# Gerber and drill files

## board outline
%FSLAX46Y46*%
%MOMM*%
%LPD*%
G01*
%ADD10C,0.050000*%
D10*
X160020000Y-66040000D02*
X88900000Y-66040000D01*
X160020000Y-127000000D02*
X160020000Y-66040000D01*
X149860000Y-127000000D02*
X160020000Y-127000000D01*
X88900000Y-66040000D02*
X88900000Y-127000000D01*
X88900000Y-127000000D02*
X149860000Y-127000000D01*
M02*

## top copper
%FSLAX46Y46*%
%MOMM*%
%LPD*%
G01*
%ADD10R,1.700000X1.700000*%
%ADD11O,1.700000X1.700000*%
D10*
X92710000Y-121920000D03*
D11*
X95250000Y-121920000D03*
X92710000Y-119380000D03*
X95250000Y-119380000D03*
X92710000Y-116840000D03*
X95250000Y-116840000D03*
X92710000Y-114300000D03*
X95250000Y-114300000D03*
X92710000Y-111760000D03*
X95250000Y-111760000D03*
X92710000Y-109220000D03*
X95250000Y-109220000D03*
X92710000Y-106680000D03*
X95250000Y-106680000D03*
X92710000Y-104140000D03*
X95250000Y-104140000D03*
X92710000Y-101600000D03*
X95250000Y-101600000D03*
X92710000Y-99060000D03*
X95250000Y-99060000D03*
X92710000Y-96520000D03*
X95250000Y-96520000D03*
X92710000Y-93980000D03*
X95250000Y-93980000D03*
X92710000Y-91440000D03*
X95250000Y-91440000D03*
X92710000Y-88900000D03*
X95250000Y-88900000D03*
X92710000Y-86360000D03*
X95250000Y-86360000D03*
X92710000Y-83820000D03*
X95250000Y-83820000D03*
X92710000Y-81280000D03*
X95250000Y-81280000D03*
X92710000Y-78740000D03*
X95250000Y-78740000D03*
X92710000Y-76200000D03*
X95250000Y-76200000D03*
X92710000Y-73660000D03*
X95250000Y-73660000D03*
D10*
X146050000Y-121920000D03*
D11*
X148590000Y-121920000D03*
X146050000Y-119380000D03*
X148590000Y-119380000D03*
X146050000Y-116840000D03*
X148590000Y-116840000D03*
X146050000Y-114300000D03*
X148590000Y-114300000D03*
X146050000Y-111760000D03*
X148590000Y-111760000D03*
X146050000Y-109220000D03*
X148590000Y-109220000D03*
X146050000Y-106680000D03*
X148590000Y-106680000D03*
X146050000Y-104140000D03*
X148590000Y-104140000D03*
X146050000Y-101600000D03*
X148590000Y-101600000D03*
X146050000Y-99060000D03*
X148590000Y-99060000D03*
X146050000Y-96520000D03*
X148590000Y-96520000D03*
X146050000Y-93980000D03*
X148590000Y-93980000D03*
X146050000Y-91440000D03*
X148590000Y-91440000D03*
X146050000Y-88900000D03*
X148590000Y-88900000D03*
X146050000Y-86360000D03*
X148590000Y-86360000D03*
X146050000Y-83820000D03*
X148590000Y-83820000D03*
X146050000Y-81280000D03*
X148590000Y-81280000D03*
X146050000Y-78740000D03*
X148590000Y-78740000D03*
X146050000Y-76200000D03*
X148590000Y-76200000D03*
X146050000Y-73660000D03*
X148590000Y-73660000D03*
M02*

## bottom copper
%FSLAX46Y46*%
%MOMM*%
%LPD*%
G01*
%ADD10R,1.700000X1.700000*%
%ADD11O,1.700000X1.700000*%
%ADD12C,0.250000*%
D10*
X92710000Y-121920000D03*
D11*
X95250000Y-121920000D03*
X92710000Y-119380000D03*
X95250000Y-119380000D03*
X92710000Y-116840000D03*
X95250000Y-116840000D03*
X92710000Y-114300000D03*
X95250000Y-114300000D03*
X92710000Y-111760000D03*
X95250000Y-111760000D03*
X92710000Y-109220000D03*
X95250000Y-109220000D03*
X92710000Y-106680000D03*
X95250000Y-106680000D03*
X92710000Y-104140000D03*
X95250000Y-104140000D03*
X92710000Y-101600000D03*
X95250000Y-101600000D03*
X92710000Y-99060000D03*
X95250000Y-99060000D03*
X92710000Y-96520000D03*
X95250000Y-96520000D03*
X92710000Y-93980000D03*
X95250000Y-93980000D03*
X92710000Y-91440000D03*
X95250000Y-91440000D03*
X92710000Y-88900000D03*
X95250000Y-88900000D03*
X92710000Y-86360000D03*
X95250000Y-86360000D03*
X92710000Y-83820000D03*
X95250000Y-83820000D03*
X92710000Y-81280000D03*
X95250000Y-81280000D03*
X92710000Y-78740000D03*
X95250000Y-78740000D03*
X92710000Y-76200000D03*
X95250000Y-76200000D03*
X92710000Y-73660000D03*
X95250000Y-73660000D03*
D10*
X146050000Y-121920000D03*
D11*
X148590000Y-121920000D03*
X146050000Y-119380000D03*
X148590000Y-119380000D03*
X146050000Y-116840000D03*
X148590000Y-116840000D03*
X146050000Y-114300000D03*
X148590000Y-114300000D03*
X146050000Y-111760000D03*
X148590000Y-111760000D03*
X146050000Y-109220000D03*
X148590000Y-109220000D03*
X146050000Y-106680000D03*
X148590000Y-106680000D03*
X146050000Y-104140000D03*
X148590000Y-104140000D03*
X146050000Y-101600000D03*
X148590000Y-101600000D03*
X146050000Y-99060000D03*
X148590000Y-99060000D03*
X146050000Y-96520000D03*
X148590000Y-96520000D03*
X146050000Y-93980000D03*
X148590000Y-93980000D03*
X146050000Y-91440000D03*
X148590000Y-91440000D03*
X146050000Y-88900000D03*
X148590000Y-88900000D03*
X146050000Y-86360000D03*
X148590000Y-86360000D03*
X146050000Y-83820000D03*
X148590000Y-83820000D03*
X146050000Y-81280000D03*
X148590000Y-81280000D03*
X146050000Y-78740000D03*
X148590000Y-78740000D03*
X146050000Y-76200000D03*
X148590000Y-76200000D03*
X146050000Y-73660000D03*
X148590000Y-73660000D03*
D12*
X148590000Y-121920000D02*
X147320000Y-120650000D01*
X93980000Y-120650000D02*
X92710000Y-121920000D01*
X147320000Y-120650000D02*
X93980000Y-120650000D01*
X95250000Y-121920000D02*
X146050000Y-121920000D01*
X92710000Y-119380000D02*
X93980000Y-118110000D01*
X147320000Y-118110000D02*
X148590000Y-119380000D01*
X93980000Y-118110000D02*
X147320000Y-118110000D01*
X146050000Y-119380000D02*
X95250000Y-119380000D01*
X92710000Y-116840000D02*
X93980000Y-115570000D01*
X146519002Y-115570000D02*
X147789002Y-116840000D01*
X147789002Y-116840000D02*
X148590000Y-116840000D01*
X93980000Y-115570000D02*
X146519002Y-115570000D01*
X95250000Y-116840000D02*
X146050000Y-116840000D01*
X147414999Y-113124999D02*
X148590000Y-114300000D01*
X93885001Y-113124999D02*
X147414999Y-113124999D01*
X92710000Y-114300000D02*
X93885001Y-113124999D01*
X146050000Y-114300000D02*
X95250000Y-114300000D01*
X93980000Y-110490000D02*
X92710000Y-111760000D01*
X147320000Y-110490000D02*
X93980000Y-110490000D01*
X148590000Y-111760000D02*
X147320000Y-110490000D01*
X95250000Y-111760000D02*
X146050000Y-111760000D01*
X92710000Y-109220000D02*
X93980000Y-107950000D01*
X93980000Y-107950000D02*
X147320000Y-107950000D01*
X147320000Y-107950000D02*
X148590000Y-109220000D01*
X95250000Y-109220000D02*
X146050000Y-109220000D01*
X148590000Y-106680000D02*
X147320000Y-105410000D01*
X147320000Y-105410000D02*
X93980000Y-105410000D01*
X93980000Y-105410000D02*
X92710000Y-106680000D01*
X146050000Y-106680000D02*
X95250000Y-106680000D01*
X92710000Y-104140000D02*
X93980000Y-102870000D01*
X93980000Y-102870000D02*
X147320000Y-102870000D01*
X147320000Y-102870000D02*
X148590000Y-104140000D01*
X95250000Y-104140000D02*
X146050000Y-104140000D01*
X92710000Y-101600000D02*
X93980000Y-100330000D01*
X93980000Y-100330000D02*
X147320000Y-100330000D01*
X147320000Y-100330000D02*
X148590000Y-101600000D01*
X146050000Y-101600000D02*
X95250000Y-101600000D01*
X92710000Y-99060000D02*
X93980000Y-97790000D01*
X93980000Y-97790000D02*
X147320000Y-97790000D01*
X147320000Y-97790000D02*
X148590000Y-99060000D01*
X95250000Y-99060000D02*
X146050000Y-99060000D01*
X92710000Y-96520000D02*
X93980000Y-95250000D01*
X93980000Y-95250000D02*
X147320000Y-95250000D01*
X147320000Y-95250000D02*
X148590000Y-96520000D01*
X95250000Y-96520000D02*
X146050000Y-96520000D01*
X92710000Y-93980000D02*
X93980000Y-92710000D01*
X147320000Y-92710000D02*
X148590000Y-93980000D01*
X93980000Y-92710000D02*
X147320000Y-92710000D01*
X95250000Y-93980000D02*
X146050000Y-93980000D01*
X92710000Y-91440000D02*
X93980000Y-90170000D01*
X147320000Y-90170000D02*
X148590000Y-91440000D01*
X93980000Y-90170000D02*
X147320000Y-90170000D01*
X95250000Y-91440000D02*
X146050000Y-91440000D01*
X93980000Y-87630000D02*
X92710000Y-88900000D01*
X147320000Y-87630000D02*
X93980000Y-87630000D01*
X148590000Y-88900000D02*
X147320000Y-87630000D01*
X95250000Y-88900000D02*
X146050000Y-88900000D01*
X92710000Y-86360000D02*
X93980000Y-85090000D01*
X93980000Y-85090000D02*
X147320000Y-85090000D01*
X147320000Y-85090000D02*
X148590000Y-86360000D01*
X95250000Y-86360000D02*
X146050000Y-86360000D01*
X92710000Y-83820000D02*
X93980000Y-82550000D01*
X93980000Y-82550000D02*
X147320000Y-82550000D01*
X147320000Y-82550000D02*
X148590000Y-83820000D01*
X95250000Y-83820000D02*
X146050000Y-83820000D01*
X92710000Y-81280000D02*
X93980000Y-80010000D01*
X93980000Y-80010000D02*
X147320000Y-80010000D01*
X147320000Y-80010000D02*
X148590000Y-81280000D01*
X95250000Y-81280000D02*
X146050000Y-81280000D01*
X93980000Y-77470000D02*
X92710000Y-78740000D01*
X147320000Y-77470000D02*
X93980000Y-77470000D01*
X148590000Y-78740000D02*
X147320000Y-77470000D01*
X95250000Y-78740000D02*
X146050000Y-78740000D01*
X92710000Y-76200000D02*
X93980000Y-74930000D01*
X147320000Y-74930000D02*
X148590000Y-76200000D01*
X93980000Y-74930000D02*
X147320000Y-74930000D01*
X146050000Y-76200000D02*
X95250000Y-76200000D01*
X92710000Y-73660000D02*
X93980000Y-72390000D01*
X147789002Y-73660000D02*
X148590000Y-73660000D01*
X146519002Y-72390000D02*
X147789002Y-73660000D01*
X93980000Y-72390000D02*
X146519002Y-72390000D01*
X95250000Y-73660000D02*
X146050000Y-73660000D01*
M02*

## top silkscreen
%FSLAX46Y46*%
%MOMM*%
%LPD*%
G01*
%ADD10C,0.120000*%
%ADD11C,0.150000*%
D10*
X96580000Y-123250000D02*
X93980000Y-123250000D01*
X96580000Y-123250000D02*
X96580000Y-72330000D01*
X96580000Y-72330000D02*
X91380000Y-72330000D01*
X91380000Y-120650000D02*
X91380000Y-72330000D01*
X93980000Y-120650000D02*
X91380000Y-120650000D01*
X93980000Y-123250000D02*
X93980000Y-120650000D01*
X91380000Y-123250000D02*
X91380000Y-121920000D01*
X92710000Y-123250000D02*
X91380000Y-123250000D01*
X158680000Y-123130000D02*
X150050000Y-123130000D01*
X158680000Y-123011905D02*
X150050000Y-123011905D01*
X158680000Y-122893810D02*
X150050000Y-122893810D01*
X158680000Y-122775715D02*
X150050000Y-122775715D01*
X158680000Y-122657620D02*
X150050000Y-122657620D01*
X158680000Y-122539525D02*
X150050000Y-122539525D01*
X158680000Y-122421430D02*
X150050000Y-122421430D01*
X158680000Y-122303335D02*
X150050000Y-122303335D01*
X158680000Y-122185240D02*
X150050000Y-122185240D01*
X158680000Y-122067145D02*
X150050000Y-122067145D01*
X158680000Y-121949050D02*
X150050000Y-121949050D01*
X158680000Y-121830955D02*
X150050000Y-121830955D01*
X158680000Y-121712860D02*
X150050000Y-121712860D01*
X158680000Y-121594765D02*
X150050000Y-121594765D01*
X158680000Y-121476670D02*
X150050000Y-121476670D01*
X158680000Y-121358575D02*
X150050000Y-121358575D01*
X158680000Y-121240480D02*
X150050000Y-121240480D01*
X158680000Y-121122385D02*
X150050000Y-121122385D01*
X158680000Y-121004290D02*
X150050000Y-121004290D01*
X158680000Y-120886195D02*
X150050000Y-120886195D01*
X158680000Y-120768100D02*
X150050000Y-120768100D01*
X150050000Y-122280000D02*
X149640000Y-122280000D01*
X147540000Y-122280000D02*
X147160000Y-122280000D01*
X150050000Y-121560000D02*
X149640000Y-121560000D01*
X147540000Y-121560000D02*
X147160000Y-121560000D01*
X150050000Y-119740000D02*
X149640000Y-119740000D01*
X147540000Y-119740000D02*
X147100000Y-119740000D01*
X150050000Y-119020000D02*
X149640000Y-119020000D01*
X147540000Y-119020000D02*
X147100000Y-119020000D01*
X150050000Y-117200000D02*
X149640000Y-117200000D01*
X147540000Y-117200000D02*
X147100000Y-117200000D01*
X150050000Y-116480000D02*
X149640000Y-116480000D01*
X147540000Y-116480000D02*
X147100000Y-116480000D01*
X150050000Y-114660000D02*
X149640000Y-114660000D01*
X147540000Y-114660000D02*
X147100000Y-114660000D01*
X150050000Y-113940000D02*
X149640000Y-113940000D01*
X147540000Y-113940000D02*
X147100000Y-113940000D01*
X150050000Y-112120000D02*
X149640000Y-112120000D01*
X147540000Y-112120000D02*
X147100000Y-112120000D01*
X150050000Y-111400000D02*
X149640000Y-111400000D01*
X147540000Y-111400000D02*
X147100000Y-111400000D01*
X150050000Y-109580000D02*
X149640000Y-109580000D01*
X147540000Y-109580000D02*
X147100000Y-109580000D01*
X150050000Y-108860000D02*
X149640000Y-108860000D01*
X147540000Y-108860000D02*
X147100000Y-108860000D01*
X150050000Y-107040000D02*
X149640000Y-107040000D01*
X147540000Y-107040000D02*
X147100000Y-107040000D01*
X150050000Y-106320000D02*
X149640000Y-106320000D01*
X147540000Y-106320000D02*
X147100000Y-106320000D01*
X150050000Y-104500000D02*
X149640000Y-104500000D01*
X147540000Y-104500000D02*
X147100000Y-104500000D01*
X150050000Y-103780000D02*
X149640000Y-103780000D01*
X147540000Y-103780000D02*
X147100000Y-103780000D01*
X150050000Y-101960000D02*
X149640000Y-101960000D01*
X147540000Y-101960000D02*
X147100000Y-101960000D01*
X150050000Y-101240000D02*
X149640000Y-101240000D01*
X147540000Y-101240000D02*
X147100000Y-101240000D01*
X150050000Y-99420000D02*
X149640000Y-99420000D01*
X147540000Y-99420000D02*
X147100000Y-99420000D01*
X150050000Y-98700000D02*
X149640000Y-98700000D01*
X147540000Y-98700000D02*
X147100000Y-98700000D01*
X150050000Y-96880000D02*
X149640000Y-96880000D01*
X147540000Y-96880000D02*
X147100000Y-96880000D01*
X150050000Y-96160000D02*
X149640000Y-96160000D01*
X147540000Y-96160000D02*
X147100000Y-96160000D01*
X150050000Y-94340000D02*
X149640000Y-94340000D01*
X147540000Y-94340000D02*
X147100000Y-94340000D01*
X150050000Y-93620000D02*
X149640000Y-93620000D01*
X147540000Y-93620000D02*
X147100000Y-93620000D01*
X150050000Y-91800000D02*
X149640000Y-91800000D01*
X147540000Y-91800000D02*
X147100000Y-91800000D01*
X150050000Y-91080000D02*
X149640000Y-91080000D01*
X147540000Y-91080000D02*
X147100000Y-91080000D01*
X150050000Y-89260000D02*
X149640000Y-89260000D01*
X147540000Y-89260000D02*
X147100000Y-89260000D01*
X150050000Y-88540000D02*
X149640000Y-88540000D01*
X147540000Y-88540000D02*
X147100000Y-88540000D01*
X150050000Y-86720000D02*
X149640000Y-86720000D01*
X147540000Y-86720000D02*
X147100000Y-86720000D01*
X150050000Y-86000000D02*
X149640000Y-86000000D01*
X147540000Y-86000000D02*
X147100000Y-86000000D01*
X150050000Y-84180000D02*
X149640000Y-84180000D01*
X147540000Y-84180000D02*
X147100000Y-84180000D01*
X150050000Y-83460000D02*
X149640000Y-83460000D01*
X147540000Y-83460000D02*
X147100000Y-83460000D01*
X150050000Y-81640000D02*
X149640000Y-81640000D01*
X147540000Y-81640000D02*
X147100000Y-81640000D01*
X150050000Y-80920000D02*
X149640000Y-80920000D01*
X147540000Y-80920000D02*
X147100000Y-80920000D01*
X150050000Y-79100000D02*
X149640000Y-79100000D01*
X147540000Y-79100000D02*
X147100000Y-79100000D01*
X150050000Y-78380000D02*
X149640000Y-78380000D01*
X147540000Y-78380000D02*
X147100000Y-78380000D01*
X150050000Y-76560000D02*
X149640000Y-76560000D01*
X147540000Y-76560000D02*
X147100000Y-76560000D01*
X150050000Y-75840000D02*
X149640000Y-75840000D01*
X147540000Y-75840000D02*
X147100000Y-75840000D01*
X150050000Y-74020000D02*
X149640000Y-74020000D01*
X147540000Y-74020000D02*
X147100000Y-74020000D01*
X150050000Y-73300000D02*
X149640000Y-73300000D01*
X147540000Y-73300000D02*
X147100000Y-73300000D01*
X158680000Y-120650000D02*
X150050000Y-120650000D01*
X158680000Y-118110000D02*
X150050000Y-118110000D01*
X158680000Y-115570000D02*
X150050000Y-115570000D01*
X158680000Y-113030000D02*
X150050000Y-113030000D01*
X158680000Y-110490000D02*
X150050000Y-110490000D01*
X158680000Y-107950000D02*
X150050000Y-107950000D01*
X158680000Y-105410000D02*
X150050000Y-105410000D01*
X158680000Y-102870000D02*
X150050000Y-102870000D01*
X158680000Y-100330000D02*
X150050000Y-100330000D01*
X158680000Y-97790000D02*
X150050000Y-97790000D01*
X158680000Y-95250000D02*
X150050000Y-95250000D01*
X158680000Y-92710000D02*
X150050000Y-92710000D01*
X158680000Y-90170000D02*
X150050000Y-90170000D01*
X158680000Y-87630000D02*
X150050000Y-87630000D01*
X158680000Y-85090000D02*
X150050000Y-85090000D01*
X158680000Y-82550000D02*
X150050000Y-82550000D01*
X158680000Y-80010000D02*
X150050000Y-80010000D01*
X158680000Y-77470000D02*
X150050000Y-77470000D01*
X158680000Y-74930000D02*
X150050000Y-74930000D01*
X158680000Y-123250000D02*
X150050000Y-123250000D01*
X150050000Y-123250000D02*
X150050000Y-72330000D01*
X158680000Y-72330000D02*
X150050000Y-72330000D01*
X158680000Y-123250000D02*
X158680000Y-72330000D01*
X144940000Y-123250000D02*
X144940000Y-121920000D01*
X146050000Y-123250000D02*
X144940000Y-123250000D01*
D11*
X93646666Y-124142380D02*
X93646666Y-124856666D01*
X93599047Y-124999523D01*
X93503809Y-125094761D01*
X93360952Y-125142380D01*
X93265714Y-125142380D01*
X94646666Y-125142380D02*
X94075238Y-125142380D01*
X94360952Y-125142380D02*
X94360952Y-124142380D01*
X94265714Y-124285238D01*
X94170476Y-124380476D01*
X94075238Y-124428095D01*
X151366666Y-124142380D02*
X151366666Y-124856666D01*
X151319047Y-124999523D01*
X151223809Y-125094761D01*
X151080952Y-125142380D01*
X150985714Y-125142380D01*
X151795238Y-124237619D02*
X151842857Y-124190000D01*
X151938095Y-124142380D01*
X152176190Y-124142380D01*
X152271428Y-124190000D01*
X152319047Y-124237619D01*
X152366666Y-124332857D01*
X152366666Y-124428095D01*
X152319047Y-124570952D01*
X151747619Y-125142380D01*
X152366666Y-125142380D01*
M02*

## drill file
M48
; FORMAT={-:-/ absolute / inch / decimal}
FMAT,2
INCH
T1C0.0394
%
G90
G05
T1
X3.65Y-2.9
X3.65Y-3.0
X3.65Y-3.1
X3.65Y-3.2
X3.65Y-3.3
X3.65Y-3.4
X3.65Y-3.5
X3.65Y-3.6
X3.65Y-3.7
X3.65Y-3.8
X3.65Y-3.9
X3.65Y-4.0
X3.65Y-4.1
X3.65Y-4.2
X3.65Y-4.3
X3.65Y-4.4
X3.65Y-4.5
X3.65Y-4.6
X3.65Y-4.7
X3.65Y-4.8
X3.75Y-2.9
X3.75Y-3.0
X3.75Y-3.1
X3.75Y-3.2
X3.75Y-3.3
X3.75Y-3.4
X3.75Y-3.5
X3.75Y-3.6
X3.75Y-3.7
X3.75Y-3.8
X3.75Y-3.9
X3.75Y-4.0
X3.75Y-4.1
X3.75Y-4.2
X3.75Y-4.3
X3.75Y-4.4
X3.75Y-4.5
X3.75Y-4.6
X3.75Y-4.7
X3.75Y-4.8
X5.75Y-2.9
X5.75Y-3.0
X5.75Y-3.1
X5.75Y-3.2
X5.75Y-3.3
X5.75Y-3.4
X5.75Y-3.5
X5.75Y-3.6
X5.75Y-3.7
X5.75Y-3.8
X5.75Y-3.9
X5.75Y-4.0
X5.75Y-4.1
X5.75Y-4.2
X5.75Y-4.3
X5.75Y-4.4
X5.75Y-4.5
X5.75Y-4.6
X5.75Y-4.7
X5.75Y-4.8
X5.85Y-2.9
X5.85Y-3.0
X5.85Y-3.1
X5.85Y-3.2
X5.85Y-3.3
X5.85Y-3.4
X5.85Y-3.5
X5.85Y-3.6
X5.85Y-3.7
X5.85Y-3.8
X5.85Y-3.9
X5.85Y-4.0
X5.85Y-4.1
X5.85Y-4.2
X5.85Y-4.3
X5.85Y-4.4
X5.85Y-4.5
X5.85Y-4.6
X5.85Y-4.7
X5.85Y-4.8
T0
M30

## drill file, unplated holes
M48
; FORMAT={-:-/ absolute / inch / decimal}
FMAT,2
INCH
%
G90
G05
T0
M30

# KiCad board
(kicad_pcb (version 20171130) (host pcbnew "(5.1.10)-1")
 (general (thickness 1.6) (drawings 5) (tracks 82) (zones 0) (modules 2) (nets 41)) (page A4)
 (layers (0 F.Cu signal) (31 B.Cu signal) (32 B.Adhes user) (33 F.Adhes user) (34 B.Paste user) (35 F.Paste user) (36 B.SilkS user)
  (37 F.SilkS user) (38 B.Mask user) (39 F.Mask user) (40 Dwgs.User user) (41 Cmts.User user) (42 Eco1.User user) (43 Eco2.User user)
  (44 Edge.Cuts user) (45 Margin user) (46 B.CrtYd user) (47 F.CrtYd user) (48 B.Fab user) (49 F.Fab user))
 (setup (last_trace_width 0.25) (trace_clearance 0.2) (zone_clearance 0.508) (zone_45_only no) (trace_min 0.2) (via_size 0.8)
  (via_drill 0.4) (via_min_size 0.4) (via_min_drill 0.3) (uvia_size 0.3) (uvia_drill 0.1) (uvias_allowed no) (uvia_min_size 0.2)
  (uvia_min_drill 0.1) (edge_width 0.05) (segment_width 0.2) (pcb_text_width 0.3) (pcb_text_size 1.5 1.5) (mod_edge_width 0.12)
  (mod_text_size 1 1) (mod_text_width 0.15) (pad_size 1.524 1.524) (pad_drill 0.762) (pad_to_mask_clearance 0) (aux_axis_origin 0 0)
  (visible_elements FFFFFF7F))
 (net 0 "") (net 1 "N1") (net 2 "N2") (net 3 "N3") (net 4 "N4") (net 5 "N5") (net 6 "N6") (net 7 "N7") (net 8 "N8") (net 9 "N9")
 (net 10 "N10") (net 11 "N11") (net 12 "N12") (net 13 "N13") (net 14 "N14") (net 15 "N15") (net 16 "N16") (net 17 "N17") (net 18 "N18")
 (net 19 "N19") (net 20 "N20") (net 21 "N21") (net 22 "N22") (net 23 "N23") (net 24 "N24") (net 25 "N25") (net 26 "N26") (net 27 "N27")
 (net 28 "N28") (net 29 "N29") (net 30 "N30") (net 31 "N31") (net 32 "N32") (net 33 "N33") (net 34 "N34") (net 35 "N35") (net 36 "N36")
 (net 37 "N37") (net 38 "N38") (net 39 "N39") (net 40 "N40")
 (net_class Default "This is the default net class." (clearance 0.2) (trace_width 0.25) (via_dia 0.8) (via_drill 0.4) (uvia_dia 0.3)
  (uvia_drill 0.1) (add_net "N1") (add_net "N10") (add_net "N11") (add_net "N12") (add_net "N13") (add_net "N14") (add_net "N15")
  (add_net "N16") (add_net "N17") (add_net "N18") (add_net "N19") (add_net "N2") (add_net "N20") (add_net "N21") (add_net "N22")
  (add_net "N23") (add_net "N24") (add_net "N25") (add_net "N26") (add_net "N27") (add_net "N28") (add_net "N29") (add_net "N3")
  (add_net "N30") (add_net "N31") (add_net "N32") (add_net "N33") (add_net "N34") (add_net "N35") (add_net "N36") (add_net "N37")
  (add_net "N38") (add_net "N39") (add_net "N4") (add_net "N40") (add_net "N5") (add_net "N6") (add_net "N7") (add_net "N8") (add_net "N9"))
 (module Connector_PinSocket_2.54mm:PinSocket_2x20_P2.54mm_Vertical (layer F.Cu) (at 92.71 121.92 180)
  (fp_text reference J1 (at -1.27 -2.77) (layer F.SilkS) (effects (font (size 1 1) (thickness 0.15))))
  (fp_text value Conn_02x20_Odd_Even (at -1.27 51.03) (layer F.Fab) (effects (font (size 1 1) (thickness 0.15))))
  (fp_line (start 0 -1.33) (end 1.33 -1.33) (layer F.SilkS) (width 0.12))
  (fp_line (start 1.33 -1.33) (end 1.33 0) (layer F.SilkS) (width 0.12))
  (fp_line (start -1.27 -1.33) (end -1.27 1.27) (layer F.SilkS) (width 0.12))
  (fp_line (start -1.27 1.27) (end 1.33 1.27) (layer F.SilkS) (width 0.12))
  (fp_line (start 1.33 1.27) (end 1.33 49.59) (layer F.SilkS) (width 0.12))
  (fp_line (start -3.87 49.59) (end 1.33 49.59) (layer F.SilkS) (width 0.12))
  (fp_line (start -3.87 -1.33) (end -3.87 49.59) (layer F.SilkS) (width 0.12))
  (fp_line (start -3.87 -1.33) (end -1.27 -1.33) (layer F.SilkS) (width 0.12))
  (pad 1 thru_hole rect (at 0 0 180) (size 1.7 1.7) (drill 1) (layers *.Cu *.Mask) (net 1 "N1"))
  (pad 2 thru_hole oval (at -2.54 0 180) (size 1.7 1.7) (drill 1) (layers *.Cu *.Mask) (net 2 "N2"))
  (pad 3 thru_hole oval (at 0 2.54 180) (size 1.7 1.7) (drill 1) (layers *.Cu *.Mask) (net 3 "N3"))
  (pad 4 thru_hole oval (at -2.54 2.54 180) (size 1.7 1.7) (drill 1) (layers *.Cu *.Mask) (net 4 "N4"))
  (pad 5 thru_hole oval (at 0 5.08 180) (size 1.7 1.7) (drill 1) (layers *.Cu *.Mask) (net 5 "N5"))
  (pad 6 thru_hole oval (at -2.54 5.08 180) (size 1.7 1.7) (drill 1) (layers *.Cu *.Mask) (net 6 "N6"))
  (pad 7 thru_hole oval (at 0 7.62 180) (size 1.7 1.7) (drill 1) (layers *.Cu *.Mask) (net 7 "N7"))
  (pad 8 thru_hole oval (at -2.54 7.62 180) (size 1.7 1.7) (drill 1) (layers *.Cu *.Mask) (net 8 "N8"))
  (pad 9 thru_hole oval (at 0 10.16 180) (size 1.7 1.7) (drill 1) (layers *.Cu *.Mask) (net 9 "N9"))
  (pad 10 thru_hole oval (at -2.54 10.16 180) (size 1.7 1.7) (drill 1) (layers *.Cu *.Mask) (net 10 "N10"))
  (pad 11 thru_hole oval (at 0 12.7 180) (size 1.7 1.7) (drill 1) (layers *.Cu *.Mask) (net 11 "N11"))
  (pad 12 thru_hole oval (at -2.54 12.7 180) (size 1.7 1.7) (drill 1) (layers *.Cu *.Mask) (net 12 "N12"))
  (pad 13 thru_hole oval (at 0 15.24 180) (size 1.7 1.7) (drill 1) (layers *.Cu *.Mask) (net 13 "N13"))
  (pad 14 thru_hole oval (at -2.54 15.24 180) (size 1.7 1.7) (drill 1) (layers *.Cu *.Mask) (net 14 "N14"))
  (pad 15 thru_hole oval (at 0 17.78 180) (size 1.7 1.7) (drill 1) (layers *.Cu *.Mask) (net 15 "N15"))
  (pad 16 thru_hole oval (at -2.54 17.78 180) (size 1.7 1.7) (drill 1) (layers *.Cu *.Mask) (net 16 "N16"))
  (pad 17 thru_hole oval (at 0 20.32 180) (size 1.7 1.7) (drill 1) (layers *.Cu *.Mask) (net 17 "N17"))
  (pad 18 thru_hole oval (at -2.54 20.32 180) (size 1.7 1.7) (drill 1) (layers *.Cu *.Mask) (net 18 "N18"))
  (pad 19 thru_hole oval (at 0 22.86 180) (size 1.7 1.7) (drill 1) (layers *.Cu *.Mask) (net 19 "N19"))
  (pad 20 thru_hole oval (at -2.54 22.86 180) (size 1.7 1.7) (drill 1) (layers *.Cu *.Mask) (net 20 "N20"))
  (pad 21 thru_hole oval (at 0 25.4 180) (size 1.7 1.7) (drill 1) (layers *.Cu *.Mask) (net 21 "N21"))
  (pad 22 thru_hole oval (at -2.54 25.4 180) (size 1.7 1.7) (drill 1) (layers *.Cu *.Mask) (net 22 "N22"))
  (pad 23 thru_hole oval (at 0 27.94 180) (size 1.7 1.7) (drill 1) (layers *.Cu *.Mask) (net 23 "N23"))
  (pad 24 thru_hole oval (at -2.54 27.94 180) (size 1.7 1.7) (drill 1) (layers *.Cu *.Mask) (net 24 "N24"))
  (pad 25 thru_hole oval (at 0 30.48 180) (size 1.7 1.7) (drill 1) (layers *.Cu *.Mask) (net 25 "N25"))
  (pad 26 thru_hole oval (at -2.54 30.48 180) (size 1.7 1.7) (drill 1) (layers *.Cu *.Mask) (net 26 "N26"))
  (pad 27 thru_hole oval (at 0 33.02 180) (size 1.7 1.7) (drill 1) (layers *.Cu *.Mask) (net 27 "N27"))
  (pad 28 thru_hole oval (at -2.54 33.02 180) (size 1.7 1.7) (drill 1) (layers *.Cu *.Mask) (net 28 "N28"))
  (pad 29 thru_hole oval (at 0 35.56 180) (size 1.7 1.7) (drill 1) (layers *.Cu *.Mask) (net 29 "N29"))
  (pad 30 thru_hole oval (at -2.54 35.56 180) (size 1.7 1.7) (drill 1) (layers *.Cu *.Mask) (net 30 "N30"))
  (pad 31 thru_hole oval (at 0 38.1 180) (size 1.7 1.7) (drill 1) (layers *.Cu *.Mask) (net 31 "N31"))
  (pad 32 thru_hole oval (at -2.54 38.1 180) (size 1.7 1.7) (drill 1) (layers *.Cu *.Mask) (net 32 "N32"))
  (pad 33 thru_hole oval (at 0 40.64 180) (size 1.7 1.7) (drill 1) (layers *.Cu *.Mask) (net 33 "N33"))
  (pad 34 thru_hole oval (at -2.54 40.64 180) (size 1.7 1.7) (drill 1) (layers *.Cu *.Mask) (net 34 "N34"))
  (pad 35 thru_hole oval (at 0 43.18 180) (size 1.7 1.7) (drill 1) (layers *.Cu *.Mask) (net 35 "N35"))
  (pad 36 thru_hole oval (at -2.54 43.18 180) (size 1.7 1.7) (drill 1) (layers *.Cu *.Mask) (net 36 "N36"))
  (pad 37 thru_hole oval (at 0 45.72 180) (size 1.7 1.7) (drill 1) (layers *.Cu *.Mask) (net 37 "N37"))
  (pad 38 thru_hole oval (at -2.54 45.72 180) (size 1.7 1.7) (drill 1) (layers *.Cu *.Mask) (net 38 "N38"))
  (pad 39 thru_hole oval (at 0 48.26 180) (size 1.7 1.7) (drill 1) (layers *.Cu *.Mask) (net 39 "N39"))
  (pad 40 thru_hole oval (at -2.54 48.26 180) (size 1.7 1.7) (drill 1) (layers *.Cu *.Mask) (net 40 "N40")))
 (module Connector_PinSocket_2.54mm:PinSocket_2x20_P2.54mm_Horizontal (layer F.Cu) (at 146.05 121.92 180)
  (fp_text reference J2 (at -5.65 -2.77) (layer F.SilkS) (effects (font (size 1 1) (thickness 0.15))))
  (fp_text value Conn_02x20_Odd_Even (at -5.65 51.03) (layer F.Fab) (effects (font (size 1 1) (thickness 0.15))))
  (fp_line (start 0 -1.33) (end 1.11 -1.33) (layer F.SilkS) (width 0.12))
  (fp_line (start 1.11 -1.33) (end 1.11 0) (layer F.SilkS) (width 0.12))
  (fp_line (start -12.63 -1.33) (end -12.63 49.59) (layer F.SilkS) (width 0.12))
  (fp_line (start -12.63 49.59) (end -4 49.59) (layer F.SilkS) (width 0.12))
  (fp_line (start -4 -1.33) (end -4 49.59) (layer F.SilkS) (width 0.12))
  (fp_line (start -12.63 -1.33) (end -4 -1.33) (layer F.SilkS) (width 0.12))
  (fp_line (start -12.63 46.99) (end -4 46.99) (layer F.SilkS) (width 0.12))
  (fp_line (start -12.63 44.45) (end -4 44.45) (layer F.SilkS) (width 0.12))
  (fp_line (start -12.63 41.91) (end -4 41.91) (layer F.SilkS) (width 0.12))
  (fp_line (start -12.63 39.37) (end -4 39.37) (layer F.SilkS) (width 0.12))
  (fp_line (start -12.63 36.83) (end -4 36.83) (layer F.SilkS) (width 0.12))
  (fp_line (start -12.63 34.29) (end -4 34.29) (layer F.SilkS) (width 0.12))
  (fp_line (start -12.63 31.75) (end -4 31.75) (layer F.SilkS) (width 0.12))
  (fp_line (start -12.63 29.21) (end -4 29.21) (layer F.SilkS) (width 0.12))
  (fp_line (start -12.63 26.67) (end -4 26.67) (layer F.SilkS) (width 0.12))
  (fp_line (start -12.63 24.13) (end -4 24.13) (layer F.SilkS) (width 0.12))
  (fp_line (start -12.63 21.59) (end -4 21.59) (layer F.SilkS) (width 0.12))
  (fp_line (start -12.63 19.05) (end -4 19.05) (layer F.SilkS) (width 0.12))
  (fp_line (start -12.63 16.51) (end -4 16.51) (layer F.SilkS) (width 0.12))
  (fp_line (start -12.63 13.97) (end -4 13.97) (layer F.SilkS) (width 0.12))
  (fp_line (start -12.63 11.43) (end -4 11.43) (layer F.SilkS) (width 0.12))
  (fp_line (start -12.63 8.89) (end -4 8.89) (layer F.SilkS) (width 0.12))
  (fp_line (start -12.63 6.35) (end -4 6.35) (layer F.SilkS) (width 0.12))
  (fp_line (start -12.63 3.81) (end -4 3.81) (layer F.SilkS) (width 0.12))
  (fp_line (start -12.63 1.27) (end -4 1.27) (layer F.SilkS) (width 0.12))
  (fp_line (start -1.49 48.62) (end -1.05 48.62) (layer F.SilkS) (width 0.12))
  (fp_line (start -4 48.62) (end -3.59 48.62) (layer F.SilkS) (width 0.12))
  (fp_line (start -1.49 47.9) (end -1.05 47.9) (layer F.SilkS) (width 0.12))
  (fp_line (start -4 47.9) (end -3.59 47.9) (layer F.SilkS) (width 0.12))
  (fp_line (start -1.49 46.08) (end -1.05 46.08) (layer F.SilkS) (width 0.12))
  (fp_line (start -4 46.08) (end -3.59 46.08) (layer F.SilkS) (width 0.12))
  (fp_line (start -1.49 45.36) (end -1.05 45.36) (layer F.SilkS) (width 0.12))
  (fp_line (start -4 45.36) (end -3.59 45.36) (layer F.SilkS) (width 0.12))
  (fp_line (start -1.49 43.54) (end -1.05 43.54) (layer F.SilkS) (width 0.12))
  (fp_line (start -4 43.54) (end -3.59 43.54) (layer F.SilkS) (width 0.12))
  (fp_line (start -1.49 42.82) (end -1.05 42.82) (layer F.SilkS) (width 0.12))
  (fp_line (start -4 42.82) (end -3.59 42.82) (layer F.SilkS) (width 0.12))
  (fp_line (start -1.49 41) (end -1.05 41) (layer F.SilkS) (width 0.12))
  (fp_line (start -4 41) (end -3.59 41) (layer F.SilkS) (width 0.12))
  (fp_line (start -1.49 40.28) (end -1.05 40.28) (layer F.SilkS) (width 0.12))
  (fp_line (start -4 40.28) (end -3.59 40.28) (layer F.SilkS) (width 0.12))
  (fp_line (start -1.49 38.46) (end -1.05 38.46) (layer F.SilkS) (width 0.12))
  (fp_line (start -4 38.46) (end -3.59 38.46) (layer F.SilkS) (width 0.12))
  (fp_line (start -1.49 37.74) (end -1.05 37.74) (layer F.SilkS) (width 0.12))
  (fp_line (start -4 37.74) (end -3.59 37.74) (layer F.SilkS) (width 0.12))
  (fp_line (start -1.49 35.92) (end -1.05 35.92) (layer F.SilkS) (width 0.12))
  (fp_line (start -4 35.92) (end -3.59 35.92) (layer F.SilkS) (width 0.12))
  (fp_line (start -1.49 35.2) (end -1.05 35.2) (layer F.SilkS) (width 0.12))
  (fp_line (start -4 35.2) (end -3.59 35.2) (layer F.SilkS) (width 0.12))
  (fp_line (start -1.49 33.38) (end -1.05 33.38) (layer F.SilkS) (width 0.12))
  (fp_line (start -4 33.38) (end -3.59 33.38) (layer F.SilkS) (width 0.12))
  (fp_line (start -1.49 32.66) (end -1.05 32.66) (layer F.SilkS) (width 0.12))
  (fp_line (start -4 32.66) (end -3.59 32.66) (layer F.SilkS) (width 0.12))
  (fp_line (start -1.49 30.84) (end -1.05 30.84) (layer F.SilkS) (width 0.12))
  (fp_line (start -4 30.84) (end -3.59 30.84) (layer F.SilkS) (width 0.12))
  (fp_line (start -1.49 30.12) (end -1.05 30.12) (layer F.SilkS) (width 0.12))
  (fp_line (start -4 30.12) (end -3.59 30.12) (layer F.SilkS) (width 0.12))
  (fp_line (start -1.49 28.3) (end -1.05 28.3) (layer F.SilkS) (width 0.12))
  (fp_line (start -4 28.3) (end -3.59 28.3) (layer F.SilkS) (width 0.12))
  (fp_line (start -1.49 27.58) (end -1.05 27.58) (layer F.SilkS) (width 0.12))
  (fp_line (start -4 27.58) (end -3.59 27.58) (layer F.SilkS) (width 0.12))
  (fp_line (start -1.49 25.76) (end -1.05 25.76) (layer F.SilkS) (width 0.12))
  (fp_line (start -4 25.76) (end -3.59 25.76) (layer F.SilkS) (width 0.12))
  (fp_line (start -1.49 25.04) (end -1.05 25.04) (layer F.SilkS) (width 0.12))
  (fp_line (start -4 25.04) (end -3.59 25.04) (layer F.SilkS) (width 0.12))
  (fp_line (start -1.49 23.22) (end -1.05 23.22) (layer F.SilkS) (width 0.12))
  (fp_line (start -4 23.22) (end -3.59 23.22) (layer F.SilkS) (width 0.12))
  (fp_line (start -1.49 22.5) (end -1.05 22.5) (layer F.SilkS) (width 0.12))
  (fp_line (start -4 22.5) (end -3.59 22.5) (layer F.SilkS) (width 0.12))
  (fp_line (start -1.49 20.68) (end -1.05 20.68) (layer F.SilkS) (width 0.12))
  (fp_line (start -4 20.68) (end -3.59 20.68) (layer F.SilkS) (width 0.12))
  (fp_line (start -1.49 19.96) (end -1.05 19.96) (layer F.SilkS) (width 0.12))
  (fp_line (start -4 19.96) (end -3.59 19.96) (layer F.SilkS) (width 0.12))
  (fp_line (start -1.49 18.14) (end -1.05 18.14) (layer F.SilkS) (width 0.12))
  (fp_line (start -4 18.14) (end -3.59 18.14) (layer F.SilkS) (width 0.12))
  (fp_line (start -1.49 17.42) (end -1.05 17.42) (layer F.SilkS) (width 0.12))
  (fp_line (start -4 17.42) (end -3.59 17.42) (layer F.SilkS) (width 0.12))
  (fp_line (start -1.49 15.6) (end -1.05 15.6) (layer F.SilkS) (width 0.12))
  (fp_line (start -4 15.6) (end -3.59 15.6) (layer F.SilkS) (width 0.12))
  (fp_line (start -1.49 14.88) (end -1.05 14.88) (layer F.SilkS) (width 0.12))
  (fp_line (start -4 14.88) (end -3.59 14.88) (layer F.SilkS) (width 0.12))
  (fp_line (start -1.49 13.06) (end -1.05 13.06) (layer F.SilkS) (width 0.12))
  (fp_line (start -4 13.06) (end -3.59 13.06) (layer F.SilkS) (width 0.12))
  (fp_line (start -1.49 12.34) (end -1.05 12.34) (layer F.SilkS) (width 0.12))
  (fp_line (start -4 12.34) (end -3.59 12.34) (layer F.SilkS) (width 0.12))
  (fp_line (start -1.49 10.52) (end -1.05 10.52) (layer F.SilkS) (width 0.12))
  (fp_line (start -4 10.52) (end -3.59 10.52) (layer F.SilkS) (width 0.12))
  (fp_line (start -1.49 9.8) (end -1.05 9.8) (layer F.SilkS) (width 0.12))
  (fp_line (start -4 9.8) (end -3.59 9.8) (layer F.SilkS) (width 0.12))
  (fp_line (start -1.49 7.98) (end -1.05 7.98) (layer F.SilkS) (width 0.12))
  (fp_line (start -4 7.98) (end -3.59 7.98) (layer F.SilkS) (width 0.12))
  (fp_line (start -1.49 7.26) (end -1.05 7.26) (layer F.SilkS) (width 0.12))
  (fp_line (start -4 7.26) (end -3.59 7.26) (layer F.SilkS) (width 0.12))
  (fp_line (start -1.49 5.44) (end -1.05 5.44) (layer F.SilkS) (width 0.12))
  (fp_line (start -4 5.44) (end -3.59 5.44) (layer F.SilkS) (width 0.12))
  (fp_line (start -1.49 4.72) (end -1.05 4.72) (layer F.SilkS) (width 0.12))
  (fp_line (start -4 4.72) (end -3.59 4.72) (layer F.SilkS) (width 0.12))
  (fp_line (start -1.49 2.9) (end -1.05 2.9) (layer F.SilkS) (width 0.12))
  (fp_line (start -4 2.9) (end -3.59 2.9) (layer F.SilkS) (width 0.12))
  (fp_line (start -1.49 2.18) (end -1.05 2.18) (layer F.SilkS) (width 0.12))
  (fp_line (start -4 2.18) (end -3.59 2.18) (layer F.SilkS) (width 0.12))
  (fp_line (start -1.49 0.36) (end -1.11 0.36) (layer F.SilkS) (width 0.12))
  (fp_line (start -4 0.36) (end -3.59 0.36) (layer F.SilkS) (width 0.12))
  (fp_line (start -1.49 -0.36) (end -1.11 -0.36) (layer F.SilkS) (width 0.12))
  (fp_line (start -4 -0.36) (end -3.59 -0.36) (layer F.SilkS) (width 0.12))
  (fp_line (start -12.63 1.1519) (end -4 1.1519) (layer F.SilkS) (width 0.12))
  (fp_line (start -12.63 1.033805) (end -4 1.033805) (layer F.SilkS) (width 0.12))
  (fp_line (start -12.63 0.91571) (end -4 0.91571) (layer F.SilkS) (width 0.12))
  (fp_line (start -12.63 0.797615) (end -4 0.797615) (layer F.SilkS) (width 0.12))
  (fp_line (start -12.63 0.67952) (end -4 0.67952) (layer F.SilkS) (width 0.12))
  (fp_line (start -12.63 0.561425) (end -4 0.561425) (layer F.SilkS) (width 0.12))
  (fp_line (start -12.63 0.44333) (end -4 0.44333) (layer F.SilkS) (width 0.12))
  (fp_line (start -12.63 0.325235) (end -4 0.325235) (layer F.SilkS) (width 0.12))
  (fp_line (start -12.63 0.20714) (end -4 0.20714) (layer F.SilkS) (width 0.12))
  (fp_line (start -12.63 0.089045) (end -4 0.089045) (layer F.SilkS) (width 0.12))
  (fp_line (start -12.63 -0.02905) (end -4 -0.02905) (layer F.SilkS) (width 0.12))
  (fp_line (start -12.63 -0.147145) (end -4 -0.147145) (layer F.SilkS) (width 0.12))
  (fp_line (start -12.63 -0.26524) (end -4 -0.26524) (layer F.SilkS) (width 0.12))
  (fp_line (start -12.63 -0.383335) (end -4 -0.383335) (layer F.SilkS) (width 0.12))
  (fp_line (start -12.63 -0.50143) (end -4 -0.50143) (layer F.SilkS) (width 0.12))
  (fp_line (start -12.63 -0.619525) (end -4 -0.619525) (layer F.SilkS) (width 0.12))
  (fp_line (start -12.63 -0.73762) (end -4 -0.73762) (layer F.SilkS) (width 0.12))
  (fp_line (start -12.63 -0.855715) (end -4 -0.855715) (layer F.SilkS) (width 0.12))
  (fp_line (start -12.63 -0.97381) (end -4 -0.97381) (layer F.SilkS) (width 0.12))
  (fp_line (start -12.63 -1.091905) (end -4 -1.091905) (layer F.SilkS) (width 0.12))
  (fp_line (start -12.63 -1.21) (end -4 -1.21) (layer F.SilkS) (width 0.12))
  (pad 1 thru_hole rect (at 0 0 180) (size 1.7 1.7) (drill 1) (layers *.Cu *.Mask) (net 2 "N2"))
  (pad 2 thru_hole oval (at -2.54 0 180) (size 1.7 1.7) (drill 1) (layers *.Cu *.Mask) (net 1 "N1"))
  (pad 3 thru_hole oval (at 0 2.54 180) (size 1.7 1.7) (drill 1) (layers *.Cu *.Mask) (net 4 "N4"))
  (pad 4 thru_hole oval (at -2.54 2.54 180) (size 1.7 1.7) (drill 1) (layers *.Cu *.Mask) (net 3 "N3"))
  (pad 5 thru_hole oval (at 0 5.08 180) (size 1.7 1.7) (drill 1) (layers *.Cu *.Mask) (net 6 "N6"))
  (pad 6 thru_hole oval (at -2.54 5.08 180) (size 1.7 1.7) (drill 1) (layers *.Cu *.Mask) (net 5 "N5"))
  (pad 7 thru_hole oval (at 0 7.62 180) (size 1.7 1.7) (drill 1) (layers *.Cu *.Mask) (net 8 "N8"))
  (pad 8 thru_hole oval (at -2.54 7.62 180) (size 1.7 1.7) (drill 1) (layers *.Cu *.Mask) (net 7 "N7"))
  (pad 9 thru_hole oval (at 0 10.16 180) (size 1.7 1.7) (drill 1) (layers *.Cu *.Mask) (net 10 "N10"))
  (pad 10 thru_hole oval (at -2.54 10.16 180) (size 1.7 1.7) (drill 1) (layers *.Cu *.Mask) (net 9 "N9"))
  (pad 11 thru_hole oval (at 0 12.7 180) (size 1.7 1.7) (drill 1) (layers *.Cu *.Mask) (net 12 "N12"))
  (pad 12 thru_hole oval (at -2.54 12.7 180) (size 1.7 1.7) (drill 1) (layers *.Cu *.Mask) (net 11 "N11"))
  (pad 13 thru_hole oval (at 0 15.24 180) (size 1.7 1.7) (drill 1) (layers *.Cu *.Mask) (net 14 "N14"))
  (pad 14 thru_hole oval (at -2.54 15.24 180) (size 1.7 1.7) (drill 1) (layers *.Cu *.Mask) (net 13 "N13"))
  (pad 15 thru_hole oval (at 0 17.78 180) (size 1.7 1.7) (drill 1) (layers *.Cu *.Mask) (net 16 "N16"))
  (pad 16 thru_hole oval (at -2.54 17.78 180) (size 1.7 1.7) (drill 1) (layers *.Cu *.Mask) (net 15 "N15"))
  (pad 17 thru_hole oval (at 0 20.32 180) (size 1.7 1.7) (drill 1) (layers *.Cu *.Mask) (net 18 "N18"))
  (pad 18 thru_hole oval (at -2.54 20.32 180) (size 1.7 1.7) (drill 1) (layers *.Cu *.Mask) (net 17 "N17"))
  (pad 19 thru_hole oval (at 0 22.86 180) (size 1.7 1.7) (drill 1) (layers *.Cu *.Mask) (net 20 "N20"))
  (pad 20 thru_hole oval (at -2.54 22.86 180) (size 1.7 1.7) (drill 1) (layers *.Cu *.Mask) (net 19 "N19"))
  (pad 21 thru_hole oval (at 0 25.4 180) (size 1.7 1.7) (drill 1) (layers *.Cu *.Mask) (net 22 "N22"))
  (pad 22 thru_hole oval (at -2.54 25.4 180) (size 1.7 1.7) (drill 1) (layers *.Cu *.Mask) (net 21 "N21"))
  (pad 23 thru_hole oval (at 0 27.94 180) (size 1.7 1.7) (drill 1) (layers *.Cu *.Mask) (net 24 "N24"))
  (pad 24 thru_hole oval (at -2.54 27.94 180) (size 1.7 1.7) (drill 1) (layers *.Cu *.Mask) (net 23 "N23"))
  (pad 25 thru_hole oval (at 0 30.48 180) (size 1.7 1.7) (drill 1) (layers *.Cu *.Mask) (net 26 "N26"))
  (pad 26 thru_hole oval (at -2.54 30.48 180) (size 1.7 1.7) (drill 1) (layers *.Cu *.Mask) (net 25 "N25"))
  (pad 27 thru_hole oval (at 0 33.02 180) (size 1.7 1.7) (drill 1) (layers *.Cu *.Mask) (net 28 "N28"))
  (pad 28 thru_hole oval (at -2.54 33.02 180) (size 1.7 1.7) (drill 1) (layers *.Cu *.Mask) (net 27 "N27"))
  (pad 29 thru_hole oval (at 0 35.56 180) (size 1.7 1.7) (drill 1) (layers *.Cu *.Mask) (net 30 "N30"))
  (pad 30 thru_hole oval (at -2.54 35.56 180) (size 1.7 1.7) (drill 1) (layers *.Cu *.Mask) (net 29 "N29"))
  (pad 31 thru_hole oval (at 0 38.1 180) (size 1.7 1.7) (drill 1) (layers *.Cu *.Mask) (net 32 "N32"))
  (pad 32 thru_hole oval (at -2.54 38.1 180) (size 1.7 1.7) (drill 1) (layers *.Cu *.Mask) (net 31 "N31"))
  (pad 33 thru_hole oval (at 0 40.64 180) (size 1.7 1.7) (drill 1) (layers *.Cu *.Mask) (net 34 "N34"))
  (pad 34 thru_hole oval (at -2.54 40.64 180) (size 1.7 1.7) (drill 1) (layers *.Cu *.Mask) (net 33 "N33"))
  (pad 35 thru_hole oval (at 0 43.18 180) (size 1.7 1.7) (drill 1) (layers *.Cu *.Mask) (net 36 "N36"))
  (pad 36 thru_hole oval (at -2.54 43.18 180) (size 1.7 1.7) (drill 1) (layers *.Cu *.Mask) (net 35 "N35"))
  (pad 37 thru_hole oval (at 0 45.72 180) (size 1.7 1.7) (drill 1) (layers *.Cu *.Mask) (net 38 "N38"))
  (pad 38 thru_hole oval (at -2.54 45.72 180) (size 1.7 1.7) (drill 1) (layers *.Cu *.Mask) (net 37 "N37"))
  (pad 39 thru_hole oval (at 0 48.26 180) (size 1.7 1.7) (drill 1) (layers *.Cu *.Mask) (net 40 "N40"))
  (pad 40 thru_hole oval (at -2.54 48.26 180) (size 1.7 1.7) (drill 1) (layers *.Cu *.Mask) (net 39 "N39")))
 (gr_line (start 160.02 66.04) (end 88.9 66.04) (layer Edge.Cuts) (width 0.05))
 (gr_line (start 160.02 127) (end 160.02 66.04) (layer Edge.Cuts) (width 0.05))
 (gr_line (start 149.86 127) (end 160.02 127) (layer Edge.Cuts) (width 0.05))
 (gr_line (start 88.9 66.04) (end 88.9 127) (layer Edge.Cuts) (width 0.05))
 (gr_line (start 88.9 127) (end 149.86 127) (layer Edge.Cuts) (width 0.05))
 (segment (start 148.59 121.92) (end 147.32 120.65) (width 0.25) (layer B.Cu) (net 1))
 (segment (start 93.98 120.65) (end 92.71 121.92) (width 0.25) (layer B.Cu) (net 1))
 (segment (start 147.32 120.65) (end 93.98 120.65) (width 0.25) (layer B.Cu) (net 1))
 (segment (start 95.25 121.92) (end 146.05 121.92) (width 0.25) (layer B.Cu) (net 2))
 (segment (start 92.71 119.38) (end 93.98 118.11) (width 0.25) (layer B.Cu) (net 3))
 (segment (start 147.32 118.11) (end 148.59 119.38) (width 0.25) (layer B.Cu) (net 3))
 (segment (start 93.98 118.11) (end 147.32 118.11) (width 0.25) (layer B.Cu) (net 3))
 (segment (start 146.05 119.38) (end 95.25 119.38) (width 0.25) (layer B.Cu) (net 4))
 (segment (start 92.71 116.84) (end 93.98 115.57) (width 0.25) (layer B.Cu) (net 5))
 (segment (start 146.519002 115.57) (end 147.789002 116.84) (width 0.25) (layer B.Cu) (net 5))
 (segment (start 147.789002 116.84) (end 148.59 116.84) (width 0.25) (layer B.Cu) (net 5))
 (segment (start 93.98 115.57) (end 146.519002 115.57) (width 0.25) (layer B.Cu) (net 5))
 (segment (start 95.25 116.84) (end 146.05 116.84) (width 0.25) (layer B.Cu) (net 6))
 (segment (start 147.414999 113.124999) (end 148.59 114.3) (width 0.25) (layer B.Cu) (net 7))
 (segment (start 93.885001 113.124999) (end 147.414999 113.124999) (width 0.25) (layer B.Cu) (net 7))
 (segment (start 92.71 114.3) (end 93.885001 113.124999) (width 0.25) (layer B.Cu) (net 7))
 (segment (start 146.05 114.3) (end 95.25 114.3) (width 0.25) (layer B.Cu) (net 8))
 (segment (start 93.98 110.49) (end 92.71 111.76) (width 0.25) (layer B.Cu) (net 9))
 (segment (start 147.32 110.49) (end 93.98 110.49) (width 0.25) (layer B.Cu) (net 9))
 (segment (start 148.59 111.76) (end 147.32 110.49) (width 0.25) (layer B.Cu) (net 9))
 (segment (start 95.25 111.76) (end 146.05 111.76) (width 0.25) (layer B.Cu) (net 10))
 (segment (start 92.71 109.22) (end 93.98 107.95) (width 0.25) (layer B.Cu) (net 11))
 (segment (start 93.98 107.95) (end 147.32 107.95) (width 0.25) (layer B.Cu) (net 11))
 (segment (start 147.32 107.95) (end 148.59 109.22) (width 0.25) (layer B.Cu) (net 11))
 (segment (start 95.25 109.22) (end 146.05 109.22) (width 0.25) (layer B.Cu) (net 12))
 (segment (start 148.59 106.68) (end 147.32 105.41) (width 0.25) (layer B.Cu) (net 13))
 (segment (start 147.32 105.41) (end 93.98 105.41) (width 0.25) (layer B.Cu) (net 13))
 (segment (start 93.98 105.41) (end 92.71 106.68) (width 0.25) (layer B.Cu) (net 13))
 (segment (start 146.05 106.68) (end 95.25 106.68) (width 0.25) (layer B.Cu) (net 14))
 (segment (start 92.71 104.14) (end 93.98 102.87) (width 0.25) (layer B.Cu) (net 15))
 (segment (start 93.98 102.87) (end 147.32 102.87) (width 0.25) (layer B.Cu) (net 15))
 (segment (start 147.32 102.87) (end 148.59 104.14) (width 0.25) (layer B.Cu) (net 15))
 (segment (start 95.25 104.14) (end 146.05 104.14) (width 0.25) (layer B.Cu) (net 16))
 (segment (start 92.71 101.6) (end 93.98 100.33) (width 0.25) (layer B.Cu) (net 17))
 (segment (start 93.98 100.33) (end 147.32 100.33) (width 0.25) (layer B.Cu) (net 17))
 (segment (start 147.32 100.33) (end 148.59 101.6) (width 0.25) (layer B.Cu) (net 17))
 (segment (start 146.05 101.6) (end 95.25 101.6) (width 0.25) (layer B.Cu) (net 18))
 (segment (start 92.71 99.06) (end 93.98 97.79) (width 0.25) (layer B.Cu) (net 19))
 (segment (start 93.98 97.79) (end 147.32 97.79) (width 0.25) (layer B.Cu) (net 19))
 (segment (start 147.32 97.79) (end 148.59 99.06) (width 0.25) (layer B.Cu) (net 19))
 (segment (start 95.25 99.06) (end 146.05 99.06) (width 0.25) (layer B.Cu) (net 20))
 (segment (start 92.71 96.52) (end 93.98 95.25) (width 0.25) (layer B.Cu) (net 21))
 (segment (start 93.98 95.25) (end 147.32 95.25) (width 0.25) (layer B.Cu) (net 21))
 (segment (start 147.32 95.25) (end 148.59 96.52) (width 0.25) (layer B.Cu) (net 21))
 (segment (start 95.25 96.52) (end 146.05 96.52) (width 0.25) (layer B.Cu) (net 22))
 (segment (start 92.71 93.98) (end 93.98 92.71) (width 0.25) (layer B.Cu) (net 23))
 (segment (start 147.32 92.71) (end 148.59 93.98) (width 0.25) (layer B.Cu) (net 23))
 (segment (start 93.98 92.71) (end 147.32 92.71) (width 0.25) (layer B.Cu) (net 23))
 (segment (start 95.25 93.98) (end 146.05 93.98) (width 0.25) (layer B.Cu) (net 24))
 (segment (start 92.71 91.44) (end 93.98 90.17) (width 0.25) (layer B.Cu) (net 25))
 (segment (start 147.32 90.17) (end 148.59 91.44) (width 0.25) (layer B.Cu) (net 25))
 (segment (start 93.98 90.17) (end 147.32 90.17) (width 0.25) (layer B.Cu) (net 25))
 (segment (start 95.25 91.44) (end 146.05 91.44) (width 0.25) (layer B.Cu) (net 26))
 (segment (start 93.98 87.63) (end 92.71 88.9) (width 0.25) (layer B.Cu) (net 27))
 (segment (start 147.32 87.63) (end 93.98 87.63) (width 0.25) (layer B.Cu) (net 27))
 (segment (start 148.59 88.9) (end 147.32 87.63) (width 0.25) (layer B.Cu) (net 27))
 (segment (start 95.25 88.9) (end 146.05 88.9) (width 0.25) (layer B.Cu) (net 28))
 (segment (start 92.71 86.36) (end 93.98 85.09) (width 0.25) (layer B.Cu) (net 29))
 (segment (start 93.98 85.09) (end 147.32 85.09) (width 0.25) (layer B.Cu) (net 29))
 (segment (start 147.32 85.09) (end 148.59 86.36) (width 0.25) (layer B.Cu) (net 29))
 (segment (start 95.25 86.36) (end 146.05 86.36) (width 0.25) (layer B.Cu) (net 30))
 (segment (start 92.71 83.82) (end 93.98 82.55) (width 0.25) (layer B.Cu) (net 31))
 (segment (start 93.98 82.55) (end 147.32 82.55) (width 0.25) (layer B.Cu) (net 31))
 (segment (start 147.32 82.55) (end 148.59 83.82) (width 0.25) (layer B.Cu) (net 31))
 (segment (start 95.25 83.82) (end 146.05 83.82) (width 0.25) (layer B.Cu) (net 32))
 (segment (start 92.71 81.28) (end 93.98 80.01) (width 0.25) (layer B.Cu) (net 33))
 (segment (start 93.98 80.01) (end 147.32 80.01) (width 0.25) (layer B.Cu) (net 33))
 (segment (start 147.32 80.01) (end 148.59 81.28) (width 0.25) (layer B.Cu) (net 33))
 (segment (start 95.25 81.28) (end 146.05 81.28) (width 0.25) (layer B.Cu) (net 34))
 (segment (start 93.98 77.47) (end 92.71 78.74) (width 0.25) (layer B.Cu) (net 35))
 (segment (start 147.32 77.47) (end 93.98 77.47) (width 0.25) (layer B.Cu) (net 35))
 (segment (start 148.59 78.74) (end 147.32 77.47) (width 0.25) (layer B.Cu) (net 35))
 (segment (start 95.25 78.74) (end 146.05 78.74) (width 0.25) (layer B.Cu) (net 36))
 (segment (start 92.71 76.2) (end 93.98 74.93) (width 0.25) (layer B.Cu) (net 37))
 (segment (start 147.32 74.93) (end 148.59 76.2) (width 0.25) (layer B.Cu) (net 37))
 (segment (start 93.98 74.93) (end 147.32 74.93) (width 0.25) (layer B.Cu) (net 37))
 (segment (start 146.05 76.2) (end 95.25 76.2) (width 0.25) (layer B.Cu) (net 38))
 (segment (start 92.71 73.66) (end 93.98 72.39) (width 0.25) (layer B.Cu) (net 39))
 (segment (start 147.789002 73.66) (end 148.59 73.66) (width 0.25) (layer B.Cu) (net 39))
 (segment (start 146.519002 72.39) (end 147.789002 73.66) (width 0.25) (layer B.Cu) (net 39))
 (segment (start 93.98 72.39) (end 146.519002 72.39) (width 0.25) (layer B.Cu) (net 39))
 (segment (start 95.25 73.66) (end 146.05 73.66) (width 0.25) (layer B.Cu) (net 40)))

